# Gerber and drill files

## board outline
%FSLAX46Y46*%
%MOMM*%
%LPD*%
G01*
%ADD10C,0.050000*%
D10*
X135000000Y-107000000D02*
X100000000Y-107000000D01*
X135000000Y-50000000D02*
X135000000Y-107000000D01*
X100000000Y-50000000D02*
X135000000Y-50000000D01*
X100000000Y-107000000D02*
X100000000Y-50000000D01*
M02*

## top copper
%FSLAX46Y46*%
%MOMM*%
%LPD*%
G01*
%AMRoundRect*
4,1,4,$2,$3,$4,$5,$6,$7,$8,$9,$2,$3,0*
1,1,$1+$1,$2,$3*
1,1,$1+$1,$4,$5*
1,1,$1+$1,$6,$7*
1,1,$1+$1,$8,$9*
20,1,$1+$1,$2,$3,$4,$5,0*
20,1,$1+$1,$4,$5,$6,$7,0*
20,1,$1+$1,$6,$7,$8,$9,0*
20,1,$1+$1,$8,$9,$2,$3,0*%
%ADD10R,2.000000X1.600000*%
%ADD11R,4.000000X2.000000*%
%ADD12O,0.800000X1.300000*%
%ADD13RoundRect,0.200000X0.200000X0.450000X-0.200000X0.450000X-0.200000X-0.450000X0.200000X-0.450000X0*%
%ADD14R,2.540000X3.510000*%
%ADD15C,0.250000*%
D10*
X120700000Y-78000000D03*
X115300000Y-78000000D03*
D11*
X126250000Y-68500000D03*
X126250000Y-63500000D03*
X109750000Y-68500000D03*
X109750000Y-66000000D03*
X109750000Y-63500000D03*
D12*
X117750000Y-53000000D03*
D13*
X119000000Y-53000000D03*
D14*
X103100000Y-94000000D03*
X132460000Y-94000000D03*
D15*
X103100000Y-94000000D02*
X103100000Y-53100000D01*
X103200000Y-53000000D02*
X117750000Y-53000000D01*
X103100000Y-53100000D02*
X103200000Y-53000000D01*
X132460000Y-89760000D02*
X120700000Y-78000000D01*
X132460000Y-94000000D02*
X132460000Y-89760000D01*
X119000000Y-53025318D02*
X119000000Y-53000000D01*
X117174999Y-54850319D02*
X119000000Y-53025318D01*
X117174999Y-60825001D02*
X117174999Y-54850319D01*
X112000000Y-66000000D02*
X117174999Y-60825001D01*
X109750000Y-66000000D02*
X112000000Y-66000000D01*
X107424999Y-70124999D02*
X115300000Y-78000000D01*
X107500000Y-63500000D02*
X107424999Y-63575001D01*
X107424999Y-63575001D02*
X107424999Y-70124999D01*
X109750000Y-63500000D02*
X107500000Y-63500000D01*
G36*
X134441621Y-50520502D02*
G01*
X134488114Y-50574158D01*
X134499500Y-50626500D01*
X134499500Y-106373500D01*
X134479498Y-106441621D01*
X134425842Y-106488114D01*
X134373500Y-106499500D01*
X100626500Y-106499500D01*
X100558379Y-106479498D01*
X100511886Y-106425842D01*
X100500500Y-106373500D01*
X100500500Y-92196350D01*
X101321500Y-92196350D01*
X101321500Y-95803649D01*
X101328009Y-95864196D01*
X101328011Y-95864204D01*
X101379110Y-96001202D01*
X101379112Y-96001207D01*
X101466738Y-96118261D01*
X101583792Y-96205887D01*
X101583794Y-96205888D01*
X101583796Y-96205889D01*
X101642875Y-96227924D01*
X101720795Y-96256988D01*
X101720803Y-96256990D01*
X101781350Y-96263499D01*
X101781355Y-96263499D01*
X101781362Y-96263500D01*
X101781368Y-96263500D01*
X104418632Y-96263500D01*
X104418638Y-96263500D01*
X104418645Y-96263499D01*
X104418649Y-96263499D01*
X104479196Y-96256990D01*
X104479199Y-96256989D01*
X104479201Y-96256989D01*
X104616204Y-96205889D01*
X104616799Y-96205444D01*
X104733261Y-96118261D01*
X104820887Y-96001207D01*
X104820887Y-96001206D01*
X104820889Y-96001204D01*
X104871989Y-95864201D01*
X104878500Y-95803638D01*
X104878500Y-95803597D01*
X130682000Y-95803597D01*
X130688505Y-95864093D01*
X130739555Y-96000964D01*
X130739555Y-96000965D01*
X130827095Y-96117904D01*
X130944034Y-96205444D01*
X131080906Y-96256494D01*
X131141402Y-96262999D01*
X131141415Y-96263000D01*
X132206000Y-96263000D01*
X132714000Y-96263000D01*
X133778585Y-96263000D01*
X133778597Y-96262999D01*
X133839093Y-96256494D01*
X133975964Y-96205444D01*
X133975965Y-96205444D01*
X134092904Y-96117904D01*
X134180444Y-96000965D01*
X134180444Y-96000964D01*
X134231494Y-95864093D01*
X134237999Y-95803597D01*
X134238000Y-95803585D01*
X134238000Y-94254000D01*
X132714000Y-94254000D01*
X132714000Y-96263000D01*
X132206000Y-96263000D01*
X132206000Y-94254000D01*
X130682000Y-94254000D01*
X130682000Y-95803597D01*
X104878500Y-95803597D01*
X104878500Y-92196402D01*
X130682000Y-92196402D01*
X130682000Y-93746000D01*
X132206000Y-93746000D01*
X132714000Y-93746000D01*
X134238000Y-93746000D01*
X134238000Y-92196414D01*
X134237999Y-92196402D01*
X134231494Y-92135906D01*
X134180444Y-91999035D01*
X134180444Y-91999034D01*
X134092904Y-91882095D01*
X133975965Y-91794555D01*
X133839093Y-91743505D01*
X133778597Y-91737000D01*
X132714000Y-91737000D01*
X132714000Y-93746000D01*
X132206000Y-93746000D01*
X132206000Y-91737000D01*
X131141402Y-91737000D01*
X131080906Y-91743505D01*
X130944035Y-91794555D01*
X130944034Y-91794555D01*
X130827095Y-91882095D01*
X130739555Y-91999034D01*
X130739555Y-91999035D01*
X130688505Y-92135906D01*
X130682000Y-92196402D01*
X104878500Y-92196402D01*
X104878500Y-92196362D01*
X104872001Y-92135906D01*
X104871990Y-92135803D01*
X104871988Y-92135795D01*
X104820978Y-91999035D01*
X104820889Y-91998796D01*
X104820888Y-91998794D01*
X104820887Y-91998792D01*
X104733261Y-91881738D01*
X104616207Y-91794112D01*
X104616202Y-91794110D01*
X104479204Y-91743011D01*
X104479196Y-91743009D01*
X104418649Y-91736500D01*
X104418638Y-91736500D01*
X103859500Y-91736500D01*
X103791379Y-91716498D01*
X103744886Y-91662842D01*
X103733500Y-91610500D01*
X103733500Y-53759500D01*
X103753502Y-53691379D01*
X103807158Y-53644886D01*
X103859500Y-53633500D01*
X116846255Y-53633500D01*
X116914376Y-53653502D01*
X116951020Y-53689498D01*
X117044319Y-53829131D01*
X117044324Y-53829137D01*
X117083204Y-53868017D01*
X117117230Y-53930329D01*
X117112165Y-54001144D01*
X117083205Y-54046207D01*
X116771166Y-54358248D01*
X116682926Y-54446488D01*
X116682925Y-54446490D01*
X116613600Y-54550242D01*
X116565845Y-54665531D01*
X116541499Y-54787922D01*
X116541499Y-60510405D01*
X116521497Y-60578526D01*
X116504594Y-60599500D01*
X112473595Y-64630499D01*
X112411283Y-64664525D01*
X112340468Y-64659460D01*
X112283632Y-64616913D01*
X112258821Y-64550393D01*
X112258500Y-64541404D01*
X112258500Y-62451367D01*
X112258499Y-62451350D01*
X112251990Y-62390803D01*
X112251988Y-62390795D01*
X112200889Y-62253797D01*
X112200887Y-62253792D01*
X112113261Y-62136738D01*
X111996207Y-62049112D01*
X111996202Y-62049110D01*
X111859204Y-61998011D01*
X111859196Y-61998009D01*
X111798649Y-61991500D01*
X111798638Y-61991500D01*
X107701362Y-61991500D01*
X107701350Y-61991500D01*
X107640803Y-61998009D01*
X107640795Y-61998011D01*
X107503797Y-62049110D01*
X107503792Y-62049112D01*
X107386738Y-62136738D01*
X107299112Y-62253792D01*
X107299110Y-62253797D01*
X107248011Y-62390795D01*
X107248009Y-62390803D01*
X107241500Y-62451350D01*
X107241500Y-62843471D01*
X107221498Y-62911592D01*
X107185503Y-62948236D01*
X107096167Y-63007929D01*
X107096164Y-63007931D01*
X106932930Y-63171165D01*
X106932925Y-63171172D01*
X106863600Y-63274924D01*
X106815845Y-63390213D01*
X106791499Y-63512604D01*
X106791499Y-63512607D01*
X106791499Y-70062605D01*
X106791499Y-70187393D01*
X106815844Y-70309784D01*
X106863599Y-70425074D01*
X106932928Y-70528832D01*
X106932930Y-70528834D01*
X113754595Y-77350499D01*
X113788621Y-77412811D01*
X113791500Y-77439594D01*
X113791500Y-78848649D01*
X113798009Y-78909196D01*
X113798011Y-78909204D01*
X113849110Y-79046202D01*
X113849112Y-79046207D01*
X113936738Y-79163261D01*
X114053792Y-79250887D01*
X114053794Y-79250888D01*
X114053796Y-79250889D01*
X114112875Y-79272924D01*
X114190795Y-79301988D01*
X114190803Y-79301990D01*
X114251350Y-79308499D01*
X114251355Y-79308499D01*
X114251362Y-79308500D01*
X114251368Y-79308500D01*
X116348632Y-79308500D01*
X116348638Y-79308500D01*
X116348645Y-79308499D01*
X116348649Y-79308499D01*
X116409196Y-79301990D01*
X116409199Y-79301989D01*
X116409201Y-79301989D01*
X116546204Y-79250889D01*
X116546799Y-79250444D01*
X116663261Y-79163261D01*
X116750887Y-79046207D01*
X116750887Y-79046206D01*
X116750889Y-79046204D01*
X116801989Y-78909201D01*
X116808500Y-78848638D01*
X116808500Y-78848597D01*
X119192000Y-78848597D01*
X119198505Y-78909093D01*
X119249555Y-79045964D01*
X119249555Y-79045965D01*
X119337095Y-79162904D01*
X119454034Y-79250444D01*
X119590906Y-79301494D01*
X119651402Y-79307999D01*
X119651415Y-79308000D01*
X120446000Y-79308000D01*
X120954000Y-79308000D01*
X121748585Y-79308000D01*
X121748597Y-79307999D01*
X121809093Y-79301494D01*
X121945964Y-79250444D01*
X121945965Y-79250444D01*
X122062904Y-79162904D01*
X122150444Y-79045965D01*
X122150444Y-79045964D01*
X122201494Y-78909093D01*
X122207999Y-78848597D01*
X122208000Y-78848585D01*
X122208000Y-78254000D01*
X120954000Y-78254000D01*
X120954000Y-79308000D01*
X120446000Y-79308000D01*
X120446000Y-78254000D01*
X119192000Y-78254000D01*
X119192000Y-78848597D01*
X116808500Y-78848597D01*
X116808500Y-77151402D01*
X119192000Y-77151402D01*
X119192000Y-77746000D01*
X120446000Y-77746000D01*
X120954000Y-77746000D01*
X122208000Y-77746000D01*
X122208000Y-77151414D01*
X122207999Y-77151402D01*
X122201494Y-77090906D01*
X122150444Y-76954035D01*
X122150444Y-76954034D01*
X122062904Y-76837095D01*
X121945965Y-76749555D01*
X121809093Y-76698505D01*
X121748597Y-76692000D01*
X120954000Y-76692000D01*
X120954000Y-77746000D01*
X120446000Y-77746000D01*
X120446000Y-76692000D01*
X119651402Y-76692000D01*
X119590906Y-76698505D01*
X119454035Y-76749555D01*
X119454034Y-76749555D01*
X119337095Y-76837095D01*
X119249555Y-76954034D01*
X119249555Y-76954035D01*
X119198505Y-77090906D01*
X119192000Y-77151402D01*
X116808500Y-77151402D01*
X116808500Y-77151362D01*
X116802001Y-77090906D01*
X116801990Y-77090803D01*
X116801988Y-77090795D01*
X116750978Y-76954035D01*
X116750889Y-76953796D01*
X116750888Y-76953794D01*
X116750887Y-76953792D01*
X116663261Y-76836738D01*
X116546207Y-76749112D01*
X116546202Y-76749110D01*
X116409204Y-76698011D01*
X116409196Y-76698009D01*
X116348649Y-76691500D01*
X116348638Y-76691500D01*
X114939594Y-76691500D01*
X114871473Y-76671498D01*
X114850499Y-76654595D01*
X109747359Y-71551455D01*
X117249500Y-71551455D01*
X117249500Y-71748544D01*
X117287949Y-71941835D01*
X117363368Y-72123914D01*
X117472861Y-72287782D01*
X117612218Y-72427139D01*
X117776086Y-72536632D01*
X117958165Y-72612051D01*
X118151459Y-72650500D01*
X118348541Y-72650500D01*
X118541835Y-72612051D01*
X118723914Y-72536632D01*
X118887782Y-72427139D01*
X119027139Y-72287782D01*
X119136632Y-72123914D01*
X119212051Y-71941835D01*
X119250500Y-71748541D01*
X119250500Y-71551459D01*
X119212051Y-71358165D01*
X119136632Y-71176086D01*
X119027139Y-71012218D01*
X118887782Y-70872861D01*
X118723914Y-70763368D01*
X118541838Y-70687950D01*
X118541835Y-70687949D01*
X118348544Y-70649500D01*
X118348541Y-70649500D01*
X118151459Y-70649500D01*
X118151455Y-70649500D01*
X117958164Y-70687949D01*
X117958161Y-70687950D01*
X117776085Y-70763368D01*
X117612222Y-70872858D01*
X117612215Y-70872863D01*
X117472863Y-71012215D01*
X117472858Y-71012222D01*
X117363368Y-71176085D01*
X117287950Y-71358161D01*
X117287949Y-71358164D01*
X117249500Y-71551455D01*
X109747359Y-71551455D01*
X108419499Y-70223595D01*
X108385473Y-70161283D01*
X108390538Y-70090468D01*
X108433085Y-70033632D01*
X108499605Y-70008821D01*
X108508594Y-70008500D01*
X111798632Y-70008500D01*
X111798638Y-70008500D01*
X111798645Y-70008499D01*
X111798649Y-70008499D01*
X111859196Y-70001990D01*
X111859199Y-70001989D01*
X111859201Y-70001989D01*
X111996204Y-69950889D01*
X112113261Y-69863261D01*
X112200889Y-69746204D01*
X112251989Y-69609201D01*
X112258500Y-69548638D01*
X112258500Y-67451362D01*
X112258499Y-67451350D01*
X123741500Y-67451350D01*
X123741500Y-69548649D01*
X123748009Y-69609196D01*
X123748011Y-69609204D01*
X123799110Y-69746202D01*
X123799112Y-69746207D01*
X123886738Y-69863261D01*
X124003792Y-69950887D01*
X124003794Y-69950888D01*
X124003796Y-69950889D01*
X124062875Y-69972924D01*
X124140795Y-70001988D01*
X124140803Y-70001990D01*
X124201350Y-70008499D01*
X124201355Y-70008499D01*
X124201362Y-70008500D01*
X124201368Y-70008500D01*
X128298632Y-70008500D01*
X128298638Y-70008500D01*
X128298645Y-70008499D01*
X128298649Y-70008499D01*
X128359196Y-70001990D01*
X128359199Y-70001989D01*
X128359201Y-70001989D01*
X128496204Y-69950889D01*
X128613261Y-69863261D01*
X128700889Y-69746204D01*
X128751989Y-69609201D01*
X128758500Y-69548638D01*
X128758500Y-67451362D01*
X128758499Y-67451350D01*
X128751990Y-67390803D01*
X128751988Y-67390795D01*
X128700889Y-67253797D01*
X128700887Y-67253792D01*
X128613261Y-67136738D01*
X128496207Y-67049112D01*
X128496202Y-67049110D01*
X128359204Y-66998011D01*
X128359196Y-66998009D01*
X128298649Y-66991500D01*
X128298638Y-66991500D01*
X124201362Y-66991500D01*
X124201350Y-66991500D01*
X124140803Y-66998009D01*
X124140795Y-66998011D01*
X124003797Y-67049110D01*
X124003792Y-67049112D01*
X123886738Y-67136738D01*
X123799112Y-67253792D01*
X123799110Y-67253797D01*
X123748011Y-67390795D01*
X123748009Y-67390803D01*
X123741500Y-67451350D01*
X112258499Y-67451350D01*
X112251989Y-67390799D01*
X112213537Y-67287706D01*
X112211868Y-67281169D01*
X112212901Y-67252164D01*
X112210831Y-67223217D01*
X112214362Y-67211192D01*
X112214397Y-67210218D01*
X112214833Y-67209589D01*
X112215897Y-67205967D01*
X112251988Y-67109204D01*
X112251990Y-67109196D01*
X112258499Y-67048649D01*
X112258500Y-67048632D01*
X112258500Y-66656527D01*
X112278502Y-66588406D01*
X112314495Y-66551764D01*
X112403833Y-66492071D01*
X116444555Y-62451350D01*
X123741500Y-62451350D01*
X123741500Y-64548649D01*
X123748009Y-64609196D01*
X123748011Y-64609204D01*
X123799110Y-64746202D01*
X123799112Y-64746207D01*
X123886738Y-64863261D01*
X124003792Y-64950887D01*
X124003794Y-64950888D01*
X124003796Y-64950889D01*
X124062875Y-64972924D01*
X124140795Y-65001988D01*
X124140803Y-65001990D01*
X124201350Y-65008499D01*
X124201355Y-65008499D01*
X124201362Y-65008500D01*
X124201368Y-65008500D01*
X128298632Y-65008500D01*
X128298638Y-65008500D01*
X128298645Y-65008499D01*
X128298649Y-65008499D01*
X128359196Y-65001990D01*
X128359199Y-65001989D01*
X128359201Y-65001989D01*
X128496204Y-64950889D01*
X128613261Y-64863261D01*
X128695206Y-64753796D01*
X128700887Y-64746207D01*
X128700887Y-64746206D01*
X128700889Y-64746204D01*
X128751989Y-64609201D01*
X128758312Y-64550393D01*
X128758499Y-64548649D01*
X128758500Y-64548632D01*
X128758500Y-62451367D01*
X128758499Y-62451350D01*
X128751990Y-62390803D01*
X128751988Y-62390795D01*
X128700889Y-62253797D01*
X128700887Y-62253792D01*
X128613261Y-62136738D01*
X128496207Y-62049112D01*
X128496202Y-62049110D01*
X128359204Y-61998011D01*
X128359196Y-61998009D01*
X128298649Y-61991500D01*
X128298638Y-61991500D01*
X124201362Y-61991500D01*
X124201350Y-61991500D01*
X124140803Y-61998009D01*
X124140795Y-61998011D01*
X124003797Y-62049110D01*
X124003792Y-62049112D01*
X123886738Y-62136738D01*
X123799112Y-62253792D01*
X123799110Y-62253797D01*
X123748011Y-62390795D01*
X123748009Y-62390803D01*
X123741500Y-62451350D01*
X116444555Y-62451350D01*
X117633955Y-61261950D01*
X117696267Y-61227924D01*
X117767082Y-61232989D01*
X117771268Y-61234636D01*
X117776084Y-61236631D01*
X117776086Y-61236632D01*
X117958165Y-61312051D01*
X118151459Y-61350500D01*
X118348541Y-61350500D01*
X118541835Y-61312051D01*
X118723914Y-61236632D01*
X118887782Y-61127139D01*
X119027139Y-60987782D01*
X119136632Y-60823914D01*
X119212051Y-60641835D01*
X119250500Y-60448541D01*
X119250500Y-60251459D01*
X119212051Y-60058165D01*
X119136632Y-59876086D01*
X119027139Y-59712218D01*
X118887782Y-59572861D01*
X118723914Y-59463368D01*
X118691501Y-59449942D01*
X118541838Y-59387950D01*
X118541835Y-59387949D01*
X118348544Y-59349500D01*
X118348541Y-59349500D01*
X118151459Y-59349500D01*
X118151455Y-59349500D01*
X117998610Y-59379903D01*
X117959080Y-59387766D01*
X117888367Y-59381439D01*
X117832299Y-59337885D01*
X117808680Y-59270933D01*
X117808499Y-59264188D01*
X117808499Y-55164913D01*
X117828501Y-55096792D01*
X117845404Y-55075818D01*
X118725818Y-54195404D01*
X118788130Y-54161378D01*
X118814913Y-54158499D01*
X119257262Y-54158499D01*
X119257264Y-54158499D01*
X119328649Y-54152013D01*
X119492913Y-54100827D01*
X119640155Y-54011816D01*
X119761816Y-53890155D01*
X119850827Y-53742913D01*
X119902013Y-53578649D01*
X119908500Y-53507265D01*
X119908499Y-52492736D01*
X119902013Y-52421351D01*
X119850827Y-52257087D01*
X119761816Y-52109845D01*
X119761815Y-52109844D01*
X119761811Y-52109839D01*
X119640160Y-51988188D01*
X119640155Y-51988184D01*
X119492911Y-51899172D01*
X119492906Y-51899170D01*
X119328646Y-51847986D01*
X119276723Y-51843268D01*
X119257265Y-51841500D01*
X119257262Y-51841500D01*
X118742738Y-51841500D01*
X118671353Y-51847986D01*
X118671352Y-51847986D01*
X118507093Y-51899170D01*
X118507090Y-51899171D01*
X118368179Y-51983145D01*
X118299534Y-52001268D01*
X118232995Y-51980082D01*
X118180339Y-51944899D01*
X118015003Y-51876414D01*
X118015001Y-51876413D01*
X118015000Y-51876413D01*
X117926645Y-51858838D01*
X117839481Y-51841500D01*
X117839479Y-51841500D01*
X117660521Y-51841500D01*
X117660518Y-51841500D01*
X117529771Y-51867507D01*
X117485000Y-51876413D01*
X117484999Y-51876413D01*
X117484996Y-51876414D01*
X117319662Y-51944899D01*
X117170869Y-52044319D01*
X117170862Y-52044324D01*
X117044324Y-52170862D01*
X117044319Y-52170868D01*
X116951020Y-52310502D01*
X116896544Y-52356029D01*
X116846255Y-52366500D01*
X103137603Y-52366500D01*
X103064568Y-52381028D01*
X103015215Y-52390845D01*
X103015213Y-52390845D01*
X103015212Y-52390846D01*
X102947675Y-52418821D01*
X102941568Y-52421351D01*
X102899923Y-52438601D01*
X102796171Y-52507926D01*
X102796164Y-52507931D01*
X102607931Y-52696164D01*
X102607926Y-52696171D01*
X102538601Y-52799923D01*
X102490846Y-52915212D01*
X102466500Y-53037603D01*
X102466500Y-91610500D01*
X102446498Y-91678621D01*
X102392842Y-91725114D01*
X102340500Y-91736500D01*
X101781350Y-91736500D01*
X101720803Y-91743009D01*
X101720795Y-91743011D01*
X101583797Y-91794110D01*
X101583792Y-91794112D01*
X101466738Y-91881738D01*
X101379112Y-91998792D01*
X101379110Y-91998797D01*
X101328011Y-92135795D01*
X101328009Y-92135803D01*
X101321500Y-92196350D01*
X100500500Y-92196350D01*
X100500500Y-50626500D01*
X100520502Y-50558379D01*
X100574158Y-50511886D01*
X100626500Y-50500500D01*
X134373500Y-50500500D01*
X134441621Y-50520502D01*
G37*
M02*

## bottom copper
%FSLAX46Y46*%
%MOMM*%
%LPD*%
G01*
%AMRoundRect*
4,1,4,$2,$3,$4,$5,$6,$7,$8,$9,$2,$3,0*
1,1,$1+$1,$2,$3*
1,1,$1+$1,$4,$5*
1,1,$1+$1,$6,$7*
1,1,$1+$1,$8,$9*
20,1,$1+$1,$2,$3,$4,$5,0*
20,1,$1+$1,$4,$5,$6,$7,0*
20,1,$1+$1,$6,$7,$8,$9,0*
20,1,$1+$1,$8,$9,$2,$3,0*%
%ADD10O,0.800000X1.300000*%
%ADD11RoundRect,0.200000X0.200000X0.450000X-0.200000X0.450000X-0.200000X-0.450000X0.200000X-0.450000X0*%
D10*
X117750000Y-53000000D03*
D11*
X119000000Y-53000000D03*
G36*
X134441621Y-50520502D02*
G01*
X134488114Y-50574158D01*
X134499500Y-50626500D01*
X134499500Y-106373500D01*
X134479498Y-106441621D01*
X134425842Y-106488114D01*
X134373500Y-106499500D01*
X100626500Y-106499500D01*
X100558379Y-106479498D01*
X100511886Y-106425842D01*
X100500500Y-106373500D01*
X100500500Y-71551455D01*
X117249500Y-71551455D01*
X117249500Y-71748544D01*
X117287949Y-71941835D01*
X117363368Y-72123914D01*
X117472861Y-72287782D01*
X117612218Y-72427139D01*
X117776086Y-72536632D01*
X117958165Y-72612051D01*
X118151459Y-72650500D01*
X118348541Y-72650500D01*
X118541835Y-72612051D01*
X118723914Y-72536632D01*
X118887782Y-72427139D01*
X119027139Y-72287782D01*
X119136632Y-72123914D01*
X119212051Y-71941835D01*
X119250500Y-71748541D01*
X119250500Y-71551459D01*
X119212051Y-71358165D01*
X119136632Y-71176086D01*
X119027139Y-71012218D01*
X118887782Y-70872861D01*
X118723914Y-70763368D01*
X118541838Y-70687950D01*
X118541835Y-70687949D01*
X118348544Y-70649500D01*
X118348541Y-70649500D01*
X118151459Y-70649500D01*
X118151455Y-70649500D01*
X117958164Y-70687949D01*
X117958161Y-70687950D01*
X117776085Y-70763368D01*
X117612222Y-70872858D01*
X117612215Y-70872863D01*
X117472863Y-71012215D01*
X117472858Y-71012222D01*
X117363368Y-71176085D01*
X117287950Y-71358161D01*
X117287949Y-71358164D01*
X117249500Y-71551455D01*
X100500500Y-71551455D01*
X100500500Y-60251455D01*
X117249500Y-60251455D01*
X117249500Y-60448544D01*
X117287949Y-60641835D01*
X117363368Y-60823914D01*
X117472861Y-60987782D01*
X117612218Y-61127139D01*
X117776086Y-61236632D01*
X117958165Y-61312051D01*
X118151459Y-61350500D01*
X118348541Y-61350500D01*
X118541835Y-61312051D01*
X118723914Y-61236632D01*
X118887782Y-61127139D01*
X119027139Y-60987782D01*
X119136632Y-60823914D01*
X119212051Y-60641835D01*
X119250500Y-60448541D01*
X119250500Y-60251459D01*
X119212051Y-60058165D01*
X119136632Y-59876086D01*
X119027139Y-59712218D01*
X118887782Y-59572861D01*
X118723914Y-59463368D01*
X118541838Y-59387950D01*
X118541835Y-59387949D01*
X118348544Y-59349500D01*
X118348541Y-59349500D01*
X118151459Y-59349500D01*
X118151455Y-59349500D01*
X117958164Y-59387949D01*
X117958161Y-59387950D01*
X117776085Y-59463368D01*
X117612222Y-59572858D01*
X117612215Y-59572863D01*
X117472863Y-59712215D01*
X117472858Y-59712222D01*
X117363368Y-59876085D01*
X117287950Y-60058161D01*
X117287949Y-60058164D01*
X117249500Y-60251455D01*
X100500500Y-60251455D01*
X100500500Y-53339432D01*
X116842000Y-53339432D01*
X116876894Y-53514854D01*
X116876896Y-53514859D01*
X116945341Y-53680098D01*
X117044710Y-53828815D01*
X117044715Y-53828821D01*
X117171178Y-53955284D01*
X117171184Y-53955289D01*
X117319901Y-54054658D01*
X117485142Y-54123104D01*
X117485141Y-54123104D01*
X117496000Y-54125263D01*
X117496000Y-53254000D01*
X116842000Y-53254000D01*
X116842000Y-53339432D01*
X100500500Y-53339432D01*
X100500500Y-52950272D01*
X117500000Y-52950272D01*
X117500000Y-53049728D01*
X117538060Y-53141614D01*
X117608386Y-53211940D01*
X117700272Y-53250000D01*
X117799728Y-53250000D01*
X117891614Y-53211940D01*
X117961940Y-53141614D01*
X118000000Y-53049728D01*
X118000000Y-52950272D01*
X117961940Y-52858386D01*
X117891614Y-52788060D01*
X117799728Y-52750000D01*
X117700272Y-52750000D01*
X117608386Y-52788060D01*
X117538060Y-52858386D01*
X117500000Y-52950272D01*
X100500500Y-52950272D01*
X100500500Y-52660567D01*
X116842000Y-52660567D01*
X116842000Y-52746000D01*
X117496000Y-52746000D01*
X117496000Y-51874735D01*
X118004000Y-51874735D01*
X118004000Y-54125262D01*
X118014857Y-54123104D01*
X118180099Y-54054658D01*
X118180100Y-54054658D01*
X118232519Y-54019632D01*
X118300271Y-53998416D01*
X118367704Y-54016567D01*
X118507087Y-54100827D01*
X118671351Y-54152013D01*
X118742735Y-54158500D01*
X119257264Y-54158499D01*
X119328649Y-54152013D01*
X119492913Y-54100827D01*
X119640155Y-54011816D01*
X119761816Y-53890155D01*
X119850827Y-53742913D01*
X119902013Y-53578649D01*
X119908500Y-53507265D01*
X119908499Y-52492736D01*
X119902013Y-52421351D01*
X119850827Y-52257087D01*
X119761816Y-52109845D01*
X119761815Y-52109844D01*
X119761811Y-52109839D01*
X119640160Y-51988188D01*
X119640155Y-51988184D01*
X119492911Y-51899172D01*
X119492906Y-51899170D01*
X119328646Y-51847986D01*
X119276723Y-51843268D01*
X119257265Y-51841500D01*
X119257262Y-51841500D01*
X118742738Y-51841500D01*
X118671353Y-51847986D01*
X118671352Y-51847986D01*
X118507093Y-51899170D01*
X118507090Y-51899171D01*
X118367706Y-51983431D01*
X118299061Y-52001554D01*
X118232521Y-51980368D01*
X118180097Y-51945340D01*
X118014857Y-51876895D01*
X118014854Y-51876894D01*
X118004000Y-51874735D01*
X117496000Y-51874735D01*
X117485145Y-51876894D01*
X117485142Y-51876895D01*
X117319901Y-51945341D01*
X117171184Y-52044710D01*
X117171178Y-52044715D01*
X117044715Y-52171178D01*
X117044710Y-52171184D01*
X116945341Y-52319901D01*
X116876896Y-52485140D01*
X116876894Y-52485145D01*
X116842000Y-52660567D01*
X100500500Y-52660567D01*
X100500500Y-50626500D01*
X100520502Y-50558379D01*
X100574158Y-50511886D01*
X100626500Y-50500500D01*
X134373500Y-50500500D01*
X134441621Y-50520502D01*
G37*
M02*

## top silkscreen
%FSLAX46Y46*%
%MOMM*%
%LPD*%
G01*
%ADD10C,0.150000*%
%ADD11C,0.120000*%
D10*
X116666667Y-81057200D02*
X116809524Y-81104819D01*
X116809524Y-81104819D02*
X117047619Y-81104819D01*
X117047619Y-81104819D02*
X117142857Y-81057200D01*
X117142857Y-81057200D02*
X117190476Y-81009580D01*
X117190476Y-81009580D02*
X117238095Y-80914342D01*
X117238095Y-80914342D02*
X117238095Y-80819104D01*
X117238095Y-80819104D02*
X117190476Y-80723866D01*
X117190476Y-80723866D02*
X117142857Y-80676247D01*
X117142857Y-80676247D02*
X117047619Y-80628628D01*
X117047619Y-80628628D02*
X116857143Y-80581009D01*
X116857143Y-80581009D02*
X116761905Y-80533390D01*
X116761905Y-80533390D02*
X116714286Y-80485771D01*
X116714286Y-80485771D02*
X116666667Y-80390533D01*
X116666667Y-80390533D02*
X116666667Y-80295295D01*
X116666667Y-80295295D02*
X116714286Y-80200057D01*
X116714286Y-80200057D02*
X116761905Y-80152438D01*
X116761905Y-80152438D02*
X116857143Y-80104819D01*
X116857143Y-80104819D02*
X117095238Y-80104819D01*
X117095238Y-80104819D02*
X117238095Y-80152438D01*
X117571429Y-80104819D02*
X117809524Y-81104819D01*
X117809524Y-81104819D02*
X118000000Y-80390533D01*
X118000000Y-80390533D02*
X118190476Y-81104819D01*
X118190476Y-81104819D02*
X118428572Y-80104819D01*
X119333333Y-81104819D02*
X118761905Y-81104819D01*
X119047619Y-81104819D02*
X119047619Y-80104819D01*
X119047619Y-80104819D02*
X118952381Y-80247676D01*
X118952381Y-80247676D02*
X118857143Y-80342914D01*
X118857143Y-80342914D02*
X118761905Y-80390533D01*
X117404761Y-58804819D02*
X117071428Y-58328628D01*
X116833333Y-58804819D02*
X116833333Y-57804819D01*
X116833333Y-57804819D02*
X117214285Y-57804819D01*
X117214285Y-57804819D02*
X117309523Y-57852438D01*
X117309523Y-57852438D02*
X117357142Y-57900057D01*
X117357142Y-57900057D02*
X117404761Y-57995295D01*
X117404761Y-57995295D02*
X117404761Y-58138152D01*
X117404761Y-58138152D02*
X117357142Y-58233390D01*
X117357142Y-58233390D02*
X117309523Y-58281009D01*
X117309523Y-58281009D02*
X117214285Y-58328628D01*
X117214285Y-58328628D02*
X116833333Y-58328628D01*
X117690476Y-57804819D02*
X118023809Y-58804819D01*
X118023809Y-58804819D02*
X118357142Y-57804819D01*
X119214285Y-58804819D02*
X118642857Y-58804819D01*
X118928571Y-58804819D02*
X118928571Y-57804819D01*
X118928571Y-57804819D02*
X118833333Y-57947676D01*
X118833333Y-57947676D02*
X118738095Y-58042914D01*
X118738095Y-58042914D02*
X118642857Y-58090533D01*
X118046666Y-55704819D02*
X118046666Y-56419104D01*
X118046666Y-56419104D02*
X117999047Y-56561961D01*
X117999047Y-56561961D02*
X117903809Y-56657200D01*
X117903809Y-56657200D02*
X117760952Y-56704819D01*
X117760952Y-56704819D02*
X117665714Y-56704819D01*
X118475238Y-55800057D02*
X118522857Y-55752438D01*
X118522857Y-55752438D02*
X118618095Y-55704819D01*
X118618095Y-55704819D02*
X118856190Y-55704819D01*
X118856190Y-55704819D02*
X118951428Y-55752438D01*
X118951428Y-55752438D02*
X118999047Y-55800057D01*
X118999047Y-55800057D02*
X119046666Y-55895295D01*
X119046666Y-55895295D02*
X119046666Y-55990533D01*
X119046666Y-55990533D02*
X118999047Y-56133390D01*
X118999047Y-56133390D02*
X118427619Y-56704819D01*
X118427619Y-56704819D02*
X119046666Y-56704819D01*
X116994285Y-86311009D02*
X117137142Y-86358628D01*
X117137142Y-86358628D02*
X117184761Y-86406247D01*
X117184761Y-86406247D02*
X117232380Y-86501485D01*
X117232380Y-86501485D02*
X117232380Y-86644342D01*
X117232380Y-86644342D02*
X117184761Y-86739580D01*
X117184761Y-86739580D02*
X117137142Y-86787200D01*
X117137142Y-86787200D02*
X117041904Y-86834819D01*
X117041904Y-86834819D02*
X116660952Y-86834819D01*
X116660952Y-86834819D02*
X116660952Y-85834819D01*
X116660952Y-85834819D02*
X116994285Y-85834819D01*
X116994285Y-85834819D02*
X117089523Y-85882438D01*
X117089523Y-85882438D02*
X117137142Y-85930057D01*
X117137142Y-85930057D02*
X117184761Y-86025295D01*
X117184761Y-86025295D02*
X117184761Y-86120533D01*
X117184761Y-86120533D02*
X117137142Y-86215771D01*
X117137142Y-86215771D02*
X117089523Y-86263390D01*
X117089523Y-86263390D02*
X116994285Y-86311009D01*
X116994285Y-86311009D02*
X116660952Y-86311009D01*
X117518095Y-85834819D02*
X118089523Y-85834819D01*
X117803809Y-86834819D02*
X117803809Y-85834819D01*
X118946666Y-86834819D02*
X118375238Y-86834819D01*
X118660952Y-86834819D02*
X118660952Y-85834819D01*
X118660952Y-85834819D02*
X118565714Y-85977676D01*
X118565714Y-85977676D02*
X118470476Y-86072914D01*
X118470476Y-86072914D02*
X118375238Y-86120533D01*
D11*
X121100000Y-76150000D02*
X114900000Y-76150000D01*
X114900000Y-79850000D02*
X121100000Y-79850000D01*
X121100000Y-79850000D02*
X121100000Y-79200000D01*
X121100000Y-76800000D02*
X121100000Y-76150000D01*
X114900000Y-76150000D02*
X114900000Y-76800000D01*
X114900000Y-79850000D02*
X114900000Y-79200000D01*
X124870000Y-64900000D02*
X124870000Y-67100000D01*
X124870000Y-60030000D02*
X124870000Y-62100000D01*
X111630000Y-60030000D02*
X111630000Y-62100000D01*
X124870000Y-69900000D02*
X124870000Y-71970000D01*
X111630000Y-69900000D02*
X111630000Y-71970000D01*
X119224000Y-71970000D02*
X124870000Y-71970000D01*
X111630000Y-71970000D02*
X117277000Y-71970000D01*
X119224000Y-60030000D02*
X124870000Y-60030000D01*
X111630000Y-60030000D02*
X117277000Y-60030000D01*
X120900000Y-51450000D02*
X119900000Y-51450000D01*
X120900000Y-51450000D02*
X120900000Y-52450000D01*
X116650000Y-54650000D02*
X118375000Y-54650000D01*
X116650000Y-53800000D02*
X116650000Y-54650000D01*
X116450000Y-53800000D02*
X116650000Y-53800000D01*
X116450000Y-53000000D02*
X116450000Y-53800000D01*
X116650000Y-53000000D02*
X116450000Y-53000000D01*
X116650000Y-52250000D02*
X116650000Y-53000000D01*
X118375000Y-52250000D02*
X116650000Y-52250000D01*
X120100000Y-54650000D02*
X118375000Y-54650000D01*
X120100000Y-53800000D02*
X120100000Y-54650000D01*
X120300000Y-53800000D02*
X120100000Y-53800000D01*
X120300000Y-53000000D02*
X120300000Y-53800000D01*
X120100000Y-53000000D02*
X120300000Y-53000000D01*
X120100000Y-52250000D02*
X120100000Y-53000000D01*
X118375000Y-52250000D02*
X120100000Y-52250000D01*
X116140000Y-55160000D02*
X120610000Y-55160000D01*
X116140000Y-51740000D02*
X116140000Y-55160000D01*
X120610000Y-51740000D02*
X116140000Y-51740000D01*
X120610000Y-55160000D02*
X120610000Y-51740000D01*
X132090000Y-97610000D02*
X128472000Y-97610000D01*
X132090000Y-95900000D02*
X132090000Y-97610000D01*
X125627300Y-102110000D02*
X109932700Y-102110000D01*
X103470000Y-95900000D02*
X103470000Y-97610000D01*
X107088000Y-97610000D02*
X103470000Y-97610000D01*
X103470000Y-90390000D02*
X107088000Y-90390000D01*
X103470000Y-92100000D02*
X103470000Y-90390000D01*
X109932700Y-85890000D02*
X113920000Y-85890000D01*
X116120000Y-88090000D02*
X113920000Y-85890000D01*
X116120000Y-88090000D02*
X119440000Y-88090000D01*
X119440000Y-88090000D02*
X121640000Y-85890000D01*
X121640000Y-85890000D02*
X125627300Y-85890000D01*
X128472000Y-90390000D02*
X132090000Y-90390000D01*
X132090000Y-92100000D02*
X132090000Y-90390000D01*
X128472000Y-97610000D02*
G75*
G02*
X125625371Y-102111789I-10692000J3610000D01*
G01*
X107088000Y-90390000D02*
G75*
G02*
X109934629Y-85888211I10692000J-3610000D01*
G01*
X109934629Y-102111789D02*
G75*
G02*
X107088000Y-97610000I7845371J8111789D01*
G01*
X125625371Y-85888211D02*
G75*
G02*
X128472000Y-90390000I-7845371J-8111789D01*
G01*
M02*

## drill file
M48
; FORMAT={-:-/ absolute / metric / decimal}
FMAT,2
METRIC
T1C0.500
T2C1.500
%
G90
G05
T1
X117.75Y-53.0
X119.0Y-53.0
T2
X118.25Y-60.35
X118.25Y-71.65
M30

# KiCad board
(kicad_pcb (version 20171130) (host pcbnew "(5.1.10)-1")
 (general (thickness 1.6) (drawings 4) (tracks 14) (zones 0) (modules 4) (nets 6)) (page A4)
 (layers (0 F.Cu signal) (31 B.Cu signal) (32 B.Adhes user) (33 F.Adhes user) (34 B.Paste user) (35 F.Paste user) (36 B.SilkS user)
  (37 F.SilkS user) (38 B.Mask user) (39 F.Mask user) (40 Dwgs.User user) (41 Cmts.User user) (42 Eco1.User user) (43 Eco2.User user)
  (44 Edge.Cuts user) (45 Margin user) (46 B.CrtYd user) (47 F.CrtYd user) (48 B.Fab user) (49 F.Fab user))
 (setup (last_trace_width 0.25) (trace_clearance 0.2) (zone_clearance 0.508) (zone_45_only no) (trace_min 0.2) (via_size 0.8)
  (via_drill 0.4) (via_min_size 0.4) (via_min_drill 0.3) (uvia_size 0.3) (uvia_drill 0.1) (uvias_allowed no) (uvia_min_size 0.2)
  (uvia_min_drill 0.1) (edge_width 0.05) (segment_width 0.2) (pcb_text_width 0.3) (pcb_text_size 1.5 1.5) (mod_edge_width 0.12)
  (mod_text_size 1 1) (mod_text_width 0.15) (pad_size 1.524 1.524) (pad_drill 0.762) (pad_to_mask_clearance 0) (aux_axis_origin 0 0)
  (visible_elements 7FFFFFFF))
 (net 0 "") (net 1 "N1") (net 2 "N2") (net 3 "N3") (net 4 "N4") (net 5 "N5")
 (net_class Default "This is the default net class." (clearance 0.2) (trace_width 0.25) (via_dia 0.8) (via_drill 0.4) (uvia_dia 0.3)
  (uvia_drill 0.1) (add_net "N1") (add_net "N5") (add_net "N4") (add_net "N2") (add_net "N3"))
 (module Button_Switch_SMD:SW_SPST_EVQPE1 (layer F.Cu) (at 118 78 180)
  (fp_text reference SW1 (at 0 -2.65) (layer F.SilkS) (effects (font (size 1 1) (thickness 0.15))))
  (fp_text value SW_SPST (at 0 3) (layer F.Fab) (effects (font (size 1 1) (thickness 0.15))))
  (fp_line (start -3.1 1.85) (end 3.1 1.85) (layer F.SilkS) (width 0.12))
  (fp_line (start 3.1 -1.85) (end -3.1 -1.85) (layer F.SilkS) (width 0.12))
  (fp_line (start -3.1 -1.85) (end -3.1 -1.2) (layer F.SilkS) (width 0.12))
  (fp_line (start -3.1 1.2) (end -3.1 1.85) (layer F.SilkS) (width 0.12))
  (fp_line (start 3.1 1.85) (end 3.1 1.2) (layer F.SilkS) (width 0.12))
  (fp_line (start 3.1 -1.85) (end 3.1 -1.2) (layer F.SilkS) (width 0.12))
  (pad 1 smd rect (at -2.7 0 180) (size 2 1.6) (layers F.Cu F.Paste F.Mask) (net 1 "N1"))
  (pad 2 smd rect (at 2.7 0 180) (size 2 1.6) (layers F.Cu F.Paste F.Mask) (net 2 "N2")))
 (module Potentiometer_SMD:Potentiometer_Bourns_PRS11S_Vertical (layer F.Cu) (at 118 66)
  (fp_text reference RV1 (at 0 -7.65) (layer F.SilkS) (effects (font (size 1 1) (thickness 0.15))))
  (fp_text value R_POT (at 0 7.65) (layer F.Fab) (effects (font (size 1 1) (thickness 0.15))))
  (fp_line (start 6.87 -1.1) (end 6.87 1.1) (layer F.SilkS) (width 0.12))
  (fp_line (start 6.87 -5.97) (end 6.87 -3.9) (layer F.SilkS) (width 0.12))
  (fp_line (start -6.37 -5.97) (end -6.37 -3.9) (layer F.SilkS) (width 0.12))
  (fp_line (start 6.87 3.9) (end 6.87 5.97) (layer F.SilkS) (width 0.12))
  (fp_line (start -6.37 3.9) (end -6.37 5.97) (layer F.SilkS) (width 0.12))
  (fp_line (start 1.224 5.97) (end 6.87 5.97) (layer F.SilkS) (width 0.12))
  (fp_line (start -6.37 5.97) (end -0.723 5.97) (layer F.SilkS) (width 0.12))
  (fp_line (start 1.224 -5.97) (end 6.87 -5.97) (layer F.SilkS) (width 0.12))
  (fp_line (start -6.37 -5.97) (end -0.723 -5.97) (layer F.SilkS) (width 0.12))
  (pad "" np_thru_hole circle (at 0.25 5.65) (size 1.5 1.5) (drill 1.5) (layers *.Cu *.Mask))
  (pad "" np_thru_hole circle (at 0.25 -5.65) (size 1.5 1.5) (drill 1.5) (layers *.Cu *.Mask))
  (pad 5 smd rect (at 8.25 2.5) (size 4 2) (layers F.Cu F.Paste F.Mask))
  (pad 4 smd rect (at 8.25 -2.5) (size 4 2) (layers F.Cu F.Paste F.Mask))
  (pad 3 smd rect (at -8.25 2.5) (size 4 2) (layers F.Cu F.Paste F.Mask) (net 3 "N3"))
  (pad 2 smd rect (at -8.25 0) (size 4 2) (layers F.Cu F.Paste F.Mask) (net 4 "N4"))
  (pad 1 smd rect (at -8.25 -2.5) (size 4 2) (layers F.Cu F.Paste F.Mask) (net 2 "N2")))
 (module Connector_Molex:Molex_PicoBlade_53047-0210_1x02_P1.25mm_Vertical (layer F.Cu) (at 119 53 180)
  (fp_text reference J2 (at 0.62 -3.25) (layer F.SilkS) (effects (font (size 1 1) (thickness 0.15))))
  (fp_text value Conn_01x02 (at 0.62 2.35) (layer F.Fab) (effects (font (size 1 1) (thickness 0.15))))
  (fp_line (start -1.9 1.55) (end -0.9 1.55) (layer F.SilkS) (width 0.12))
  (fp_line (start -1.9 1.55) (end -1.9 0.55) (layer F.SilkS) (width 0.12))
  (fp_line (start 2.35 -1.65) (end 0.625 -1.65) (layer F.SilkS) (width 0.12))
  (fp_line (start 2.35 -0.8) (end 2.35 -1.65) (layer F.SilkS) (width 0.12))
  (fp_line (start 2.55 -0.8) (end 2.35 -0.8) (layer F.SilkS) (width 0.12))
  (fp_line (start 2.55 0) (end 2.55 -0.8) (layer F.SilkS) (width 0.12))
  (fp_line (start 2.35 0) (end 2.55 0) (layer F.SilkS) (width 0.12))
  (fp_line (start 2.35 0.75) (end 2.35 0) (layer F.SilkS) (width 0.12))
  (fp_line (start 0.625 0.75) (end 2.35 0.75) (layer F.SilkS) (width 0.12))
  (fp_line (start -1.1 -1.65) (end 0.625 -1.65) (layer F.SilkS) (width 0.12))
  (fp_line (start -1.1 -0.8) (end -1.1 -1.65) (layer F.SilkS) (width 0.12))
  (fp_line (start -1.3 -0.8) (end -1.1 -0.8) (layer F.SilkS) (width 0.12))
  (fp_line (start -1.3 0) (end -1.3 -0.8) (layer F.SilkS) (width 0.12))
  (fp_line (start -1.1 0) (end -1.3 0) (layer F.SilkS) (width 0.12))
  (fp_line (start -1.1 0.75) (end -1.1 0) (layer F.SilkS) (width 0.12))
  (fp_line (start 0.625 0.75) (end -1.1 0.75) (layer F.SilkS) (width 0.12))
  (fp_line (start 2.86 -2.16) (end -1.61 -2.16) (layer F.SilkS) (width 0.12))
  (fp_line (start 2.86 1.26) (end 2.86 -2.16) (layer F.SilkS) (width 0.12))
  (fp_line (start -1.61 1.26) (end 2.86 1.26) (layer F.SilkS) (width 0.12))
  (fp_line (start -1.61 -2.16) (end -1.61 1.26) (layer F.SilkS) (width 0.12))
  (pad 2 thru_hole oval (at 1.25 0 180) (size 0.8 1.3) (drill 0.5) (layers *.Cu *.Mask) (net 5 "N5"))
  (pad 1 thru_hole roundrect (at 0 0 180) (size 0.8 1.3) (drill 0.5) (layers *.Cu *.Mask) (roundrect_rratio 0.25) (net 4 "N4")))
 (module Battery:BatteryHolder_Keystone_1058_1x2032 (layer F.Cu) (at 117.78 94 180)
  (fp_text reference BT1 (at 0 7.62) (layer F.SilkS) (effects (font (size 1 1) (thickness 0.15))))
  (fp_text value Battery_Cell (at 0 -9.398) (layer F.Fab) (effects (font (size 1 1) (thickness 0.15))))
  (fp_line (start -14.31 -3.61) (end -10.692 -3.61) (layer F.SilkS) (width 0.12))
  (fp_line (start -14.31 -1.9) (end -14.31 -3.61) (layer F.SilkS) (width 0.12))
  (fp_line (start -7.8473 -8.11) (end 7.8473 -8.11) (layer F.SilkS) (width 0.12))
  (fp_line (start 14.31 -1.9) (end 14.31 -3.61) (layer F.SilkS) (width 0.12))
  (fp_line (start 10.692 -3.61) (end 14.31 -3.61) (layer F.SilkS) (width 0.12))
  (fp_line (start 14.31 3.61) (end 10.692 3.61) (layer F.SilkS) (width 0.12))
  (fp_line (start 14.31 1.9) (end 14.31 3.61) (layer F.SilkS) (width 0.12))
  (fp_line (start 7.8473 8.11) (end 3.86 8.11) (layer F.SilkS) (width 0.12))
  (fp_line (start 1.66 5.91) (end 3.86 8.11) (layer F.SilkS) (width 0.12))
  (fp_line (start 1.66 5.91) (end -1.66 5.91) (layer F.SilkS) (width 0.12))
  (fp_line (start -1.66 5.91) (end -3.86 8.11) (layer F.SilkS) (width 0.12))
  (fp_line (start -3.86 8.11) (end -7.8473 8.11) (layer F.SilkS) (width 0.12))
  (fp_line (start -10.692 3.61) (end -14.31 3.61) (layer F.SilkS) (width 0.12))
  (fp_line (start -14.31 1.9) (end -14.31 3.61) (layer F.SilkS) (width 0.12))
  (fp_arc (start 0 0) (end -10.692 -3.61) (angle 27.3) (layer F.SilkS) (width 0.12))
  (fp_arc (start 0 0) (end 10.692 3.61) (angle 27.3) (layer F.SilkS) (width 0.12))
  (fp_arc (start 0 0) (end 10.692 -3.61) (angle -27.3) (layer F.SilkS) (width 0.12))
  (fp_arc (start 0 0) (end -10.692 3.61) (angle -27.3) (layer F.SilkS) (width 0.12))
  (pad 2 smd rect (at 14.68 0 180) (size 2.54 3.51) (layers F.Cu F.Paste F.Mask) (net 5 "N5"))
  (pad 1 smd rect (at -14.68 0 180) (size 2.54 3.51) (layers F.Cu F.Paste F.Mask) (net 1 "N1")))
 (gr_line (start 135 107) (end 100 107) (layer Edge.Cuts) (width 0.05))
 (gr_line (start 135 50) (end 135 107) (layer Edge.Cuts) (width 0.05))
 (gr_line (start 100 50) (end 135 50) (layer Edge.Cuts) (width 0.05))
 (gr_line (start 100 107) (end 100 50) (layer Edge.Cuts) (width 0.05))
 (segment (start 103.1 94) (end 103.1 53.1) (width 0.25) (layer F.Cu) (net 5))
 (segment (start 103.2 53) (end 117.75 53) (width 0.25) (layer F.Cu) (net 5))
 (segment (start 103.1 53.1) (end 103.2 53) (width 0.25) (layer F.Cu) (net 5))
 (segment (start 132.46 89.76) (end 120.7 78) (width 0.25) (layer F.Cu) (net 1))
 (segment (start 132.46 94) (end 132.46 89.76) (width 0.25) (layer F.Cu) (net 1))
 (segment (start 119 53.025318) (end 119 53) (width 0.25) (layer F.Cu) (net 4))
 (segment (start 117.174999 54.850319) (end 119 53.025318) (width 0.25) (layer F.Cu) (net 4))
 (segment (start 117.174999 60.825001) (end 117.174999 54.850319) (width 0.25) (layer F.Cu) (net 4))
 (segment (start 112 66) (end 117.174999 60.825001) (width 0.25) (layer F.Cu) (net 4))
 (segment (start 109.75 66) (end 112 66) (width 0.25) (layer F.Cu) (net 4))
 (segment (start 107.424999 70.124999) (end 115.3 78) (width 0.25) (layer F.Cu) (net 2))
 (segment (start 107.5 63.5) (end 107.424999 63.575001) (width 0.25) (layer F.Cu) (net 2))
 (segment (start 107.424999 63.575001) (end 107.424999 70.124999) (width 0.25) (layer F.Cu) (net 2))
 (segment (start 109.75 63.5) (end 107.5 63.5) (width 0.25) (layer F.Cu) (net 2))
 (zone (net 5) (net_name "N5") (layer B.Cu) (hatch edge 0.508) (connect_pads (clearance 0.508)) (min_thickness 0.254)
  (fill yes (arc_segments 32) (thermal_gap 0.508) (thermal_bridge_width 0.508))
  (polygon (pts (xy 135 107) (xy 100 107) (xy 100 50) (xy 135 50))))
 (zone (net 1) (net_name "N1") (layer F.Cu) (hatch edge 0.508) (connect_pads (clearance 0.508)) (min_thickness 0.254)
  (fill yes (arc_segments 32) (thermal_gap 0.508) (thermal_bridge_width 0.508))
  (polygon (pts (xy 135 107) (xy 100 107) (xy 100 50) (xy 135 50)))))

